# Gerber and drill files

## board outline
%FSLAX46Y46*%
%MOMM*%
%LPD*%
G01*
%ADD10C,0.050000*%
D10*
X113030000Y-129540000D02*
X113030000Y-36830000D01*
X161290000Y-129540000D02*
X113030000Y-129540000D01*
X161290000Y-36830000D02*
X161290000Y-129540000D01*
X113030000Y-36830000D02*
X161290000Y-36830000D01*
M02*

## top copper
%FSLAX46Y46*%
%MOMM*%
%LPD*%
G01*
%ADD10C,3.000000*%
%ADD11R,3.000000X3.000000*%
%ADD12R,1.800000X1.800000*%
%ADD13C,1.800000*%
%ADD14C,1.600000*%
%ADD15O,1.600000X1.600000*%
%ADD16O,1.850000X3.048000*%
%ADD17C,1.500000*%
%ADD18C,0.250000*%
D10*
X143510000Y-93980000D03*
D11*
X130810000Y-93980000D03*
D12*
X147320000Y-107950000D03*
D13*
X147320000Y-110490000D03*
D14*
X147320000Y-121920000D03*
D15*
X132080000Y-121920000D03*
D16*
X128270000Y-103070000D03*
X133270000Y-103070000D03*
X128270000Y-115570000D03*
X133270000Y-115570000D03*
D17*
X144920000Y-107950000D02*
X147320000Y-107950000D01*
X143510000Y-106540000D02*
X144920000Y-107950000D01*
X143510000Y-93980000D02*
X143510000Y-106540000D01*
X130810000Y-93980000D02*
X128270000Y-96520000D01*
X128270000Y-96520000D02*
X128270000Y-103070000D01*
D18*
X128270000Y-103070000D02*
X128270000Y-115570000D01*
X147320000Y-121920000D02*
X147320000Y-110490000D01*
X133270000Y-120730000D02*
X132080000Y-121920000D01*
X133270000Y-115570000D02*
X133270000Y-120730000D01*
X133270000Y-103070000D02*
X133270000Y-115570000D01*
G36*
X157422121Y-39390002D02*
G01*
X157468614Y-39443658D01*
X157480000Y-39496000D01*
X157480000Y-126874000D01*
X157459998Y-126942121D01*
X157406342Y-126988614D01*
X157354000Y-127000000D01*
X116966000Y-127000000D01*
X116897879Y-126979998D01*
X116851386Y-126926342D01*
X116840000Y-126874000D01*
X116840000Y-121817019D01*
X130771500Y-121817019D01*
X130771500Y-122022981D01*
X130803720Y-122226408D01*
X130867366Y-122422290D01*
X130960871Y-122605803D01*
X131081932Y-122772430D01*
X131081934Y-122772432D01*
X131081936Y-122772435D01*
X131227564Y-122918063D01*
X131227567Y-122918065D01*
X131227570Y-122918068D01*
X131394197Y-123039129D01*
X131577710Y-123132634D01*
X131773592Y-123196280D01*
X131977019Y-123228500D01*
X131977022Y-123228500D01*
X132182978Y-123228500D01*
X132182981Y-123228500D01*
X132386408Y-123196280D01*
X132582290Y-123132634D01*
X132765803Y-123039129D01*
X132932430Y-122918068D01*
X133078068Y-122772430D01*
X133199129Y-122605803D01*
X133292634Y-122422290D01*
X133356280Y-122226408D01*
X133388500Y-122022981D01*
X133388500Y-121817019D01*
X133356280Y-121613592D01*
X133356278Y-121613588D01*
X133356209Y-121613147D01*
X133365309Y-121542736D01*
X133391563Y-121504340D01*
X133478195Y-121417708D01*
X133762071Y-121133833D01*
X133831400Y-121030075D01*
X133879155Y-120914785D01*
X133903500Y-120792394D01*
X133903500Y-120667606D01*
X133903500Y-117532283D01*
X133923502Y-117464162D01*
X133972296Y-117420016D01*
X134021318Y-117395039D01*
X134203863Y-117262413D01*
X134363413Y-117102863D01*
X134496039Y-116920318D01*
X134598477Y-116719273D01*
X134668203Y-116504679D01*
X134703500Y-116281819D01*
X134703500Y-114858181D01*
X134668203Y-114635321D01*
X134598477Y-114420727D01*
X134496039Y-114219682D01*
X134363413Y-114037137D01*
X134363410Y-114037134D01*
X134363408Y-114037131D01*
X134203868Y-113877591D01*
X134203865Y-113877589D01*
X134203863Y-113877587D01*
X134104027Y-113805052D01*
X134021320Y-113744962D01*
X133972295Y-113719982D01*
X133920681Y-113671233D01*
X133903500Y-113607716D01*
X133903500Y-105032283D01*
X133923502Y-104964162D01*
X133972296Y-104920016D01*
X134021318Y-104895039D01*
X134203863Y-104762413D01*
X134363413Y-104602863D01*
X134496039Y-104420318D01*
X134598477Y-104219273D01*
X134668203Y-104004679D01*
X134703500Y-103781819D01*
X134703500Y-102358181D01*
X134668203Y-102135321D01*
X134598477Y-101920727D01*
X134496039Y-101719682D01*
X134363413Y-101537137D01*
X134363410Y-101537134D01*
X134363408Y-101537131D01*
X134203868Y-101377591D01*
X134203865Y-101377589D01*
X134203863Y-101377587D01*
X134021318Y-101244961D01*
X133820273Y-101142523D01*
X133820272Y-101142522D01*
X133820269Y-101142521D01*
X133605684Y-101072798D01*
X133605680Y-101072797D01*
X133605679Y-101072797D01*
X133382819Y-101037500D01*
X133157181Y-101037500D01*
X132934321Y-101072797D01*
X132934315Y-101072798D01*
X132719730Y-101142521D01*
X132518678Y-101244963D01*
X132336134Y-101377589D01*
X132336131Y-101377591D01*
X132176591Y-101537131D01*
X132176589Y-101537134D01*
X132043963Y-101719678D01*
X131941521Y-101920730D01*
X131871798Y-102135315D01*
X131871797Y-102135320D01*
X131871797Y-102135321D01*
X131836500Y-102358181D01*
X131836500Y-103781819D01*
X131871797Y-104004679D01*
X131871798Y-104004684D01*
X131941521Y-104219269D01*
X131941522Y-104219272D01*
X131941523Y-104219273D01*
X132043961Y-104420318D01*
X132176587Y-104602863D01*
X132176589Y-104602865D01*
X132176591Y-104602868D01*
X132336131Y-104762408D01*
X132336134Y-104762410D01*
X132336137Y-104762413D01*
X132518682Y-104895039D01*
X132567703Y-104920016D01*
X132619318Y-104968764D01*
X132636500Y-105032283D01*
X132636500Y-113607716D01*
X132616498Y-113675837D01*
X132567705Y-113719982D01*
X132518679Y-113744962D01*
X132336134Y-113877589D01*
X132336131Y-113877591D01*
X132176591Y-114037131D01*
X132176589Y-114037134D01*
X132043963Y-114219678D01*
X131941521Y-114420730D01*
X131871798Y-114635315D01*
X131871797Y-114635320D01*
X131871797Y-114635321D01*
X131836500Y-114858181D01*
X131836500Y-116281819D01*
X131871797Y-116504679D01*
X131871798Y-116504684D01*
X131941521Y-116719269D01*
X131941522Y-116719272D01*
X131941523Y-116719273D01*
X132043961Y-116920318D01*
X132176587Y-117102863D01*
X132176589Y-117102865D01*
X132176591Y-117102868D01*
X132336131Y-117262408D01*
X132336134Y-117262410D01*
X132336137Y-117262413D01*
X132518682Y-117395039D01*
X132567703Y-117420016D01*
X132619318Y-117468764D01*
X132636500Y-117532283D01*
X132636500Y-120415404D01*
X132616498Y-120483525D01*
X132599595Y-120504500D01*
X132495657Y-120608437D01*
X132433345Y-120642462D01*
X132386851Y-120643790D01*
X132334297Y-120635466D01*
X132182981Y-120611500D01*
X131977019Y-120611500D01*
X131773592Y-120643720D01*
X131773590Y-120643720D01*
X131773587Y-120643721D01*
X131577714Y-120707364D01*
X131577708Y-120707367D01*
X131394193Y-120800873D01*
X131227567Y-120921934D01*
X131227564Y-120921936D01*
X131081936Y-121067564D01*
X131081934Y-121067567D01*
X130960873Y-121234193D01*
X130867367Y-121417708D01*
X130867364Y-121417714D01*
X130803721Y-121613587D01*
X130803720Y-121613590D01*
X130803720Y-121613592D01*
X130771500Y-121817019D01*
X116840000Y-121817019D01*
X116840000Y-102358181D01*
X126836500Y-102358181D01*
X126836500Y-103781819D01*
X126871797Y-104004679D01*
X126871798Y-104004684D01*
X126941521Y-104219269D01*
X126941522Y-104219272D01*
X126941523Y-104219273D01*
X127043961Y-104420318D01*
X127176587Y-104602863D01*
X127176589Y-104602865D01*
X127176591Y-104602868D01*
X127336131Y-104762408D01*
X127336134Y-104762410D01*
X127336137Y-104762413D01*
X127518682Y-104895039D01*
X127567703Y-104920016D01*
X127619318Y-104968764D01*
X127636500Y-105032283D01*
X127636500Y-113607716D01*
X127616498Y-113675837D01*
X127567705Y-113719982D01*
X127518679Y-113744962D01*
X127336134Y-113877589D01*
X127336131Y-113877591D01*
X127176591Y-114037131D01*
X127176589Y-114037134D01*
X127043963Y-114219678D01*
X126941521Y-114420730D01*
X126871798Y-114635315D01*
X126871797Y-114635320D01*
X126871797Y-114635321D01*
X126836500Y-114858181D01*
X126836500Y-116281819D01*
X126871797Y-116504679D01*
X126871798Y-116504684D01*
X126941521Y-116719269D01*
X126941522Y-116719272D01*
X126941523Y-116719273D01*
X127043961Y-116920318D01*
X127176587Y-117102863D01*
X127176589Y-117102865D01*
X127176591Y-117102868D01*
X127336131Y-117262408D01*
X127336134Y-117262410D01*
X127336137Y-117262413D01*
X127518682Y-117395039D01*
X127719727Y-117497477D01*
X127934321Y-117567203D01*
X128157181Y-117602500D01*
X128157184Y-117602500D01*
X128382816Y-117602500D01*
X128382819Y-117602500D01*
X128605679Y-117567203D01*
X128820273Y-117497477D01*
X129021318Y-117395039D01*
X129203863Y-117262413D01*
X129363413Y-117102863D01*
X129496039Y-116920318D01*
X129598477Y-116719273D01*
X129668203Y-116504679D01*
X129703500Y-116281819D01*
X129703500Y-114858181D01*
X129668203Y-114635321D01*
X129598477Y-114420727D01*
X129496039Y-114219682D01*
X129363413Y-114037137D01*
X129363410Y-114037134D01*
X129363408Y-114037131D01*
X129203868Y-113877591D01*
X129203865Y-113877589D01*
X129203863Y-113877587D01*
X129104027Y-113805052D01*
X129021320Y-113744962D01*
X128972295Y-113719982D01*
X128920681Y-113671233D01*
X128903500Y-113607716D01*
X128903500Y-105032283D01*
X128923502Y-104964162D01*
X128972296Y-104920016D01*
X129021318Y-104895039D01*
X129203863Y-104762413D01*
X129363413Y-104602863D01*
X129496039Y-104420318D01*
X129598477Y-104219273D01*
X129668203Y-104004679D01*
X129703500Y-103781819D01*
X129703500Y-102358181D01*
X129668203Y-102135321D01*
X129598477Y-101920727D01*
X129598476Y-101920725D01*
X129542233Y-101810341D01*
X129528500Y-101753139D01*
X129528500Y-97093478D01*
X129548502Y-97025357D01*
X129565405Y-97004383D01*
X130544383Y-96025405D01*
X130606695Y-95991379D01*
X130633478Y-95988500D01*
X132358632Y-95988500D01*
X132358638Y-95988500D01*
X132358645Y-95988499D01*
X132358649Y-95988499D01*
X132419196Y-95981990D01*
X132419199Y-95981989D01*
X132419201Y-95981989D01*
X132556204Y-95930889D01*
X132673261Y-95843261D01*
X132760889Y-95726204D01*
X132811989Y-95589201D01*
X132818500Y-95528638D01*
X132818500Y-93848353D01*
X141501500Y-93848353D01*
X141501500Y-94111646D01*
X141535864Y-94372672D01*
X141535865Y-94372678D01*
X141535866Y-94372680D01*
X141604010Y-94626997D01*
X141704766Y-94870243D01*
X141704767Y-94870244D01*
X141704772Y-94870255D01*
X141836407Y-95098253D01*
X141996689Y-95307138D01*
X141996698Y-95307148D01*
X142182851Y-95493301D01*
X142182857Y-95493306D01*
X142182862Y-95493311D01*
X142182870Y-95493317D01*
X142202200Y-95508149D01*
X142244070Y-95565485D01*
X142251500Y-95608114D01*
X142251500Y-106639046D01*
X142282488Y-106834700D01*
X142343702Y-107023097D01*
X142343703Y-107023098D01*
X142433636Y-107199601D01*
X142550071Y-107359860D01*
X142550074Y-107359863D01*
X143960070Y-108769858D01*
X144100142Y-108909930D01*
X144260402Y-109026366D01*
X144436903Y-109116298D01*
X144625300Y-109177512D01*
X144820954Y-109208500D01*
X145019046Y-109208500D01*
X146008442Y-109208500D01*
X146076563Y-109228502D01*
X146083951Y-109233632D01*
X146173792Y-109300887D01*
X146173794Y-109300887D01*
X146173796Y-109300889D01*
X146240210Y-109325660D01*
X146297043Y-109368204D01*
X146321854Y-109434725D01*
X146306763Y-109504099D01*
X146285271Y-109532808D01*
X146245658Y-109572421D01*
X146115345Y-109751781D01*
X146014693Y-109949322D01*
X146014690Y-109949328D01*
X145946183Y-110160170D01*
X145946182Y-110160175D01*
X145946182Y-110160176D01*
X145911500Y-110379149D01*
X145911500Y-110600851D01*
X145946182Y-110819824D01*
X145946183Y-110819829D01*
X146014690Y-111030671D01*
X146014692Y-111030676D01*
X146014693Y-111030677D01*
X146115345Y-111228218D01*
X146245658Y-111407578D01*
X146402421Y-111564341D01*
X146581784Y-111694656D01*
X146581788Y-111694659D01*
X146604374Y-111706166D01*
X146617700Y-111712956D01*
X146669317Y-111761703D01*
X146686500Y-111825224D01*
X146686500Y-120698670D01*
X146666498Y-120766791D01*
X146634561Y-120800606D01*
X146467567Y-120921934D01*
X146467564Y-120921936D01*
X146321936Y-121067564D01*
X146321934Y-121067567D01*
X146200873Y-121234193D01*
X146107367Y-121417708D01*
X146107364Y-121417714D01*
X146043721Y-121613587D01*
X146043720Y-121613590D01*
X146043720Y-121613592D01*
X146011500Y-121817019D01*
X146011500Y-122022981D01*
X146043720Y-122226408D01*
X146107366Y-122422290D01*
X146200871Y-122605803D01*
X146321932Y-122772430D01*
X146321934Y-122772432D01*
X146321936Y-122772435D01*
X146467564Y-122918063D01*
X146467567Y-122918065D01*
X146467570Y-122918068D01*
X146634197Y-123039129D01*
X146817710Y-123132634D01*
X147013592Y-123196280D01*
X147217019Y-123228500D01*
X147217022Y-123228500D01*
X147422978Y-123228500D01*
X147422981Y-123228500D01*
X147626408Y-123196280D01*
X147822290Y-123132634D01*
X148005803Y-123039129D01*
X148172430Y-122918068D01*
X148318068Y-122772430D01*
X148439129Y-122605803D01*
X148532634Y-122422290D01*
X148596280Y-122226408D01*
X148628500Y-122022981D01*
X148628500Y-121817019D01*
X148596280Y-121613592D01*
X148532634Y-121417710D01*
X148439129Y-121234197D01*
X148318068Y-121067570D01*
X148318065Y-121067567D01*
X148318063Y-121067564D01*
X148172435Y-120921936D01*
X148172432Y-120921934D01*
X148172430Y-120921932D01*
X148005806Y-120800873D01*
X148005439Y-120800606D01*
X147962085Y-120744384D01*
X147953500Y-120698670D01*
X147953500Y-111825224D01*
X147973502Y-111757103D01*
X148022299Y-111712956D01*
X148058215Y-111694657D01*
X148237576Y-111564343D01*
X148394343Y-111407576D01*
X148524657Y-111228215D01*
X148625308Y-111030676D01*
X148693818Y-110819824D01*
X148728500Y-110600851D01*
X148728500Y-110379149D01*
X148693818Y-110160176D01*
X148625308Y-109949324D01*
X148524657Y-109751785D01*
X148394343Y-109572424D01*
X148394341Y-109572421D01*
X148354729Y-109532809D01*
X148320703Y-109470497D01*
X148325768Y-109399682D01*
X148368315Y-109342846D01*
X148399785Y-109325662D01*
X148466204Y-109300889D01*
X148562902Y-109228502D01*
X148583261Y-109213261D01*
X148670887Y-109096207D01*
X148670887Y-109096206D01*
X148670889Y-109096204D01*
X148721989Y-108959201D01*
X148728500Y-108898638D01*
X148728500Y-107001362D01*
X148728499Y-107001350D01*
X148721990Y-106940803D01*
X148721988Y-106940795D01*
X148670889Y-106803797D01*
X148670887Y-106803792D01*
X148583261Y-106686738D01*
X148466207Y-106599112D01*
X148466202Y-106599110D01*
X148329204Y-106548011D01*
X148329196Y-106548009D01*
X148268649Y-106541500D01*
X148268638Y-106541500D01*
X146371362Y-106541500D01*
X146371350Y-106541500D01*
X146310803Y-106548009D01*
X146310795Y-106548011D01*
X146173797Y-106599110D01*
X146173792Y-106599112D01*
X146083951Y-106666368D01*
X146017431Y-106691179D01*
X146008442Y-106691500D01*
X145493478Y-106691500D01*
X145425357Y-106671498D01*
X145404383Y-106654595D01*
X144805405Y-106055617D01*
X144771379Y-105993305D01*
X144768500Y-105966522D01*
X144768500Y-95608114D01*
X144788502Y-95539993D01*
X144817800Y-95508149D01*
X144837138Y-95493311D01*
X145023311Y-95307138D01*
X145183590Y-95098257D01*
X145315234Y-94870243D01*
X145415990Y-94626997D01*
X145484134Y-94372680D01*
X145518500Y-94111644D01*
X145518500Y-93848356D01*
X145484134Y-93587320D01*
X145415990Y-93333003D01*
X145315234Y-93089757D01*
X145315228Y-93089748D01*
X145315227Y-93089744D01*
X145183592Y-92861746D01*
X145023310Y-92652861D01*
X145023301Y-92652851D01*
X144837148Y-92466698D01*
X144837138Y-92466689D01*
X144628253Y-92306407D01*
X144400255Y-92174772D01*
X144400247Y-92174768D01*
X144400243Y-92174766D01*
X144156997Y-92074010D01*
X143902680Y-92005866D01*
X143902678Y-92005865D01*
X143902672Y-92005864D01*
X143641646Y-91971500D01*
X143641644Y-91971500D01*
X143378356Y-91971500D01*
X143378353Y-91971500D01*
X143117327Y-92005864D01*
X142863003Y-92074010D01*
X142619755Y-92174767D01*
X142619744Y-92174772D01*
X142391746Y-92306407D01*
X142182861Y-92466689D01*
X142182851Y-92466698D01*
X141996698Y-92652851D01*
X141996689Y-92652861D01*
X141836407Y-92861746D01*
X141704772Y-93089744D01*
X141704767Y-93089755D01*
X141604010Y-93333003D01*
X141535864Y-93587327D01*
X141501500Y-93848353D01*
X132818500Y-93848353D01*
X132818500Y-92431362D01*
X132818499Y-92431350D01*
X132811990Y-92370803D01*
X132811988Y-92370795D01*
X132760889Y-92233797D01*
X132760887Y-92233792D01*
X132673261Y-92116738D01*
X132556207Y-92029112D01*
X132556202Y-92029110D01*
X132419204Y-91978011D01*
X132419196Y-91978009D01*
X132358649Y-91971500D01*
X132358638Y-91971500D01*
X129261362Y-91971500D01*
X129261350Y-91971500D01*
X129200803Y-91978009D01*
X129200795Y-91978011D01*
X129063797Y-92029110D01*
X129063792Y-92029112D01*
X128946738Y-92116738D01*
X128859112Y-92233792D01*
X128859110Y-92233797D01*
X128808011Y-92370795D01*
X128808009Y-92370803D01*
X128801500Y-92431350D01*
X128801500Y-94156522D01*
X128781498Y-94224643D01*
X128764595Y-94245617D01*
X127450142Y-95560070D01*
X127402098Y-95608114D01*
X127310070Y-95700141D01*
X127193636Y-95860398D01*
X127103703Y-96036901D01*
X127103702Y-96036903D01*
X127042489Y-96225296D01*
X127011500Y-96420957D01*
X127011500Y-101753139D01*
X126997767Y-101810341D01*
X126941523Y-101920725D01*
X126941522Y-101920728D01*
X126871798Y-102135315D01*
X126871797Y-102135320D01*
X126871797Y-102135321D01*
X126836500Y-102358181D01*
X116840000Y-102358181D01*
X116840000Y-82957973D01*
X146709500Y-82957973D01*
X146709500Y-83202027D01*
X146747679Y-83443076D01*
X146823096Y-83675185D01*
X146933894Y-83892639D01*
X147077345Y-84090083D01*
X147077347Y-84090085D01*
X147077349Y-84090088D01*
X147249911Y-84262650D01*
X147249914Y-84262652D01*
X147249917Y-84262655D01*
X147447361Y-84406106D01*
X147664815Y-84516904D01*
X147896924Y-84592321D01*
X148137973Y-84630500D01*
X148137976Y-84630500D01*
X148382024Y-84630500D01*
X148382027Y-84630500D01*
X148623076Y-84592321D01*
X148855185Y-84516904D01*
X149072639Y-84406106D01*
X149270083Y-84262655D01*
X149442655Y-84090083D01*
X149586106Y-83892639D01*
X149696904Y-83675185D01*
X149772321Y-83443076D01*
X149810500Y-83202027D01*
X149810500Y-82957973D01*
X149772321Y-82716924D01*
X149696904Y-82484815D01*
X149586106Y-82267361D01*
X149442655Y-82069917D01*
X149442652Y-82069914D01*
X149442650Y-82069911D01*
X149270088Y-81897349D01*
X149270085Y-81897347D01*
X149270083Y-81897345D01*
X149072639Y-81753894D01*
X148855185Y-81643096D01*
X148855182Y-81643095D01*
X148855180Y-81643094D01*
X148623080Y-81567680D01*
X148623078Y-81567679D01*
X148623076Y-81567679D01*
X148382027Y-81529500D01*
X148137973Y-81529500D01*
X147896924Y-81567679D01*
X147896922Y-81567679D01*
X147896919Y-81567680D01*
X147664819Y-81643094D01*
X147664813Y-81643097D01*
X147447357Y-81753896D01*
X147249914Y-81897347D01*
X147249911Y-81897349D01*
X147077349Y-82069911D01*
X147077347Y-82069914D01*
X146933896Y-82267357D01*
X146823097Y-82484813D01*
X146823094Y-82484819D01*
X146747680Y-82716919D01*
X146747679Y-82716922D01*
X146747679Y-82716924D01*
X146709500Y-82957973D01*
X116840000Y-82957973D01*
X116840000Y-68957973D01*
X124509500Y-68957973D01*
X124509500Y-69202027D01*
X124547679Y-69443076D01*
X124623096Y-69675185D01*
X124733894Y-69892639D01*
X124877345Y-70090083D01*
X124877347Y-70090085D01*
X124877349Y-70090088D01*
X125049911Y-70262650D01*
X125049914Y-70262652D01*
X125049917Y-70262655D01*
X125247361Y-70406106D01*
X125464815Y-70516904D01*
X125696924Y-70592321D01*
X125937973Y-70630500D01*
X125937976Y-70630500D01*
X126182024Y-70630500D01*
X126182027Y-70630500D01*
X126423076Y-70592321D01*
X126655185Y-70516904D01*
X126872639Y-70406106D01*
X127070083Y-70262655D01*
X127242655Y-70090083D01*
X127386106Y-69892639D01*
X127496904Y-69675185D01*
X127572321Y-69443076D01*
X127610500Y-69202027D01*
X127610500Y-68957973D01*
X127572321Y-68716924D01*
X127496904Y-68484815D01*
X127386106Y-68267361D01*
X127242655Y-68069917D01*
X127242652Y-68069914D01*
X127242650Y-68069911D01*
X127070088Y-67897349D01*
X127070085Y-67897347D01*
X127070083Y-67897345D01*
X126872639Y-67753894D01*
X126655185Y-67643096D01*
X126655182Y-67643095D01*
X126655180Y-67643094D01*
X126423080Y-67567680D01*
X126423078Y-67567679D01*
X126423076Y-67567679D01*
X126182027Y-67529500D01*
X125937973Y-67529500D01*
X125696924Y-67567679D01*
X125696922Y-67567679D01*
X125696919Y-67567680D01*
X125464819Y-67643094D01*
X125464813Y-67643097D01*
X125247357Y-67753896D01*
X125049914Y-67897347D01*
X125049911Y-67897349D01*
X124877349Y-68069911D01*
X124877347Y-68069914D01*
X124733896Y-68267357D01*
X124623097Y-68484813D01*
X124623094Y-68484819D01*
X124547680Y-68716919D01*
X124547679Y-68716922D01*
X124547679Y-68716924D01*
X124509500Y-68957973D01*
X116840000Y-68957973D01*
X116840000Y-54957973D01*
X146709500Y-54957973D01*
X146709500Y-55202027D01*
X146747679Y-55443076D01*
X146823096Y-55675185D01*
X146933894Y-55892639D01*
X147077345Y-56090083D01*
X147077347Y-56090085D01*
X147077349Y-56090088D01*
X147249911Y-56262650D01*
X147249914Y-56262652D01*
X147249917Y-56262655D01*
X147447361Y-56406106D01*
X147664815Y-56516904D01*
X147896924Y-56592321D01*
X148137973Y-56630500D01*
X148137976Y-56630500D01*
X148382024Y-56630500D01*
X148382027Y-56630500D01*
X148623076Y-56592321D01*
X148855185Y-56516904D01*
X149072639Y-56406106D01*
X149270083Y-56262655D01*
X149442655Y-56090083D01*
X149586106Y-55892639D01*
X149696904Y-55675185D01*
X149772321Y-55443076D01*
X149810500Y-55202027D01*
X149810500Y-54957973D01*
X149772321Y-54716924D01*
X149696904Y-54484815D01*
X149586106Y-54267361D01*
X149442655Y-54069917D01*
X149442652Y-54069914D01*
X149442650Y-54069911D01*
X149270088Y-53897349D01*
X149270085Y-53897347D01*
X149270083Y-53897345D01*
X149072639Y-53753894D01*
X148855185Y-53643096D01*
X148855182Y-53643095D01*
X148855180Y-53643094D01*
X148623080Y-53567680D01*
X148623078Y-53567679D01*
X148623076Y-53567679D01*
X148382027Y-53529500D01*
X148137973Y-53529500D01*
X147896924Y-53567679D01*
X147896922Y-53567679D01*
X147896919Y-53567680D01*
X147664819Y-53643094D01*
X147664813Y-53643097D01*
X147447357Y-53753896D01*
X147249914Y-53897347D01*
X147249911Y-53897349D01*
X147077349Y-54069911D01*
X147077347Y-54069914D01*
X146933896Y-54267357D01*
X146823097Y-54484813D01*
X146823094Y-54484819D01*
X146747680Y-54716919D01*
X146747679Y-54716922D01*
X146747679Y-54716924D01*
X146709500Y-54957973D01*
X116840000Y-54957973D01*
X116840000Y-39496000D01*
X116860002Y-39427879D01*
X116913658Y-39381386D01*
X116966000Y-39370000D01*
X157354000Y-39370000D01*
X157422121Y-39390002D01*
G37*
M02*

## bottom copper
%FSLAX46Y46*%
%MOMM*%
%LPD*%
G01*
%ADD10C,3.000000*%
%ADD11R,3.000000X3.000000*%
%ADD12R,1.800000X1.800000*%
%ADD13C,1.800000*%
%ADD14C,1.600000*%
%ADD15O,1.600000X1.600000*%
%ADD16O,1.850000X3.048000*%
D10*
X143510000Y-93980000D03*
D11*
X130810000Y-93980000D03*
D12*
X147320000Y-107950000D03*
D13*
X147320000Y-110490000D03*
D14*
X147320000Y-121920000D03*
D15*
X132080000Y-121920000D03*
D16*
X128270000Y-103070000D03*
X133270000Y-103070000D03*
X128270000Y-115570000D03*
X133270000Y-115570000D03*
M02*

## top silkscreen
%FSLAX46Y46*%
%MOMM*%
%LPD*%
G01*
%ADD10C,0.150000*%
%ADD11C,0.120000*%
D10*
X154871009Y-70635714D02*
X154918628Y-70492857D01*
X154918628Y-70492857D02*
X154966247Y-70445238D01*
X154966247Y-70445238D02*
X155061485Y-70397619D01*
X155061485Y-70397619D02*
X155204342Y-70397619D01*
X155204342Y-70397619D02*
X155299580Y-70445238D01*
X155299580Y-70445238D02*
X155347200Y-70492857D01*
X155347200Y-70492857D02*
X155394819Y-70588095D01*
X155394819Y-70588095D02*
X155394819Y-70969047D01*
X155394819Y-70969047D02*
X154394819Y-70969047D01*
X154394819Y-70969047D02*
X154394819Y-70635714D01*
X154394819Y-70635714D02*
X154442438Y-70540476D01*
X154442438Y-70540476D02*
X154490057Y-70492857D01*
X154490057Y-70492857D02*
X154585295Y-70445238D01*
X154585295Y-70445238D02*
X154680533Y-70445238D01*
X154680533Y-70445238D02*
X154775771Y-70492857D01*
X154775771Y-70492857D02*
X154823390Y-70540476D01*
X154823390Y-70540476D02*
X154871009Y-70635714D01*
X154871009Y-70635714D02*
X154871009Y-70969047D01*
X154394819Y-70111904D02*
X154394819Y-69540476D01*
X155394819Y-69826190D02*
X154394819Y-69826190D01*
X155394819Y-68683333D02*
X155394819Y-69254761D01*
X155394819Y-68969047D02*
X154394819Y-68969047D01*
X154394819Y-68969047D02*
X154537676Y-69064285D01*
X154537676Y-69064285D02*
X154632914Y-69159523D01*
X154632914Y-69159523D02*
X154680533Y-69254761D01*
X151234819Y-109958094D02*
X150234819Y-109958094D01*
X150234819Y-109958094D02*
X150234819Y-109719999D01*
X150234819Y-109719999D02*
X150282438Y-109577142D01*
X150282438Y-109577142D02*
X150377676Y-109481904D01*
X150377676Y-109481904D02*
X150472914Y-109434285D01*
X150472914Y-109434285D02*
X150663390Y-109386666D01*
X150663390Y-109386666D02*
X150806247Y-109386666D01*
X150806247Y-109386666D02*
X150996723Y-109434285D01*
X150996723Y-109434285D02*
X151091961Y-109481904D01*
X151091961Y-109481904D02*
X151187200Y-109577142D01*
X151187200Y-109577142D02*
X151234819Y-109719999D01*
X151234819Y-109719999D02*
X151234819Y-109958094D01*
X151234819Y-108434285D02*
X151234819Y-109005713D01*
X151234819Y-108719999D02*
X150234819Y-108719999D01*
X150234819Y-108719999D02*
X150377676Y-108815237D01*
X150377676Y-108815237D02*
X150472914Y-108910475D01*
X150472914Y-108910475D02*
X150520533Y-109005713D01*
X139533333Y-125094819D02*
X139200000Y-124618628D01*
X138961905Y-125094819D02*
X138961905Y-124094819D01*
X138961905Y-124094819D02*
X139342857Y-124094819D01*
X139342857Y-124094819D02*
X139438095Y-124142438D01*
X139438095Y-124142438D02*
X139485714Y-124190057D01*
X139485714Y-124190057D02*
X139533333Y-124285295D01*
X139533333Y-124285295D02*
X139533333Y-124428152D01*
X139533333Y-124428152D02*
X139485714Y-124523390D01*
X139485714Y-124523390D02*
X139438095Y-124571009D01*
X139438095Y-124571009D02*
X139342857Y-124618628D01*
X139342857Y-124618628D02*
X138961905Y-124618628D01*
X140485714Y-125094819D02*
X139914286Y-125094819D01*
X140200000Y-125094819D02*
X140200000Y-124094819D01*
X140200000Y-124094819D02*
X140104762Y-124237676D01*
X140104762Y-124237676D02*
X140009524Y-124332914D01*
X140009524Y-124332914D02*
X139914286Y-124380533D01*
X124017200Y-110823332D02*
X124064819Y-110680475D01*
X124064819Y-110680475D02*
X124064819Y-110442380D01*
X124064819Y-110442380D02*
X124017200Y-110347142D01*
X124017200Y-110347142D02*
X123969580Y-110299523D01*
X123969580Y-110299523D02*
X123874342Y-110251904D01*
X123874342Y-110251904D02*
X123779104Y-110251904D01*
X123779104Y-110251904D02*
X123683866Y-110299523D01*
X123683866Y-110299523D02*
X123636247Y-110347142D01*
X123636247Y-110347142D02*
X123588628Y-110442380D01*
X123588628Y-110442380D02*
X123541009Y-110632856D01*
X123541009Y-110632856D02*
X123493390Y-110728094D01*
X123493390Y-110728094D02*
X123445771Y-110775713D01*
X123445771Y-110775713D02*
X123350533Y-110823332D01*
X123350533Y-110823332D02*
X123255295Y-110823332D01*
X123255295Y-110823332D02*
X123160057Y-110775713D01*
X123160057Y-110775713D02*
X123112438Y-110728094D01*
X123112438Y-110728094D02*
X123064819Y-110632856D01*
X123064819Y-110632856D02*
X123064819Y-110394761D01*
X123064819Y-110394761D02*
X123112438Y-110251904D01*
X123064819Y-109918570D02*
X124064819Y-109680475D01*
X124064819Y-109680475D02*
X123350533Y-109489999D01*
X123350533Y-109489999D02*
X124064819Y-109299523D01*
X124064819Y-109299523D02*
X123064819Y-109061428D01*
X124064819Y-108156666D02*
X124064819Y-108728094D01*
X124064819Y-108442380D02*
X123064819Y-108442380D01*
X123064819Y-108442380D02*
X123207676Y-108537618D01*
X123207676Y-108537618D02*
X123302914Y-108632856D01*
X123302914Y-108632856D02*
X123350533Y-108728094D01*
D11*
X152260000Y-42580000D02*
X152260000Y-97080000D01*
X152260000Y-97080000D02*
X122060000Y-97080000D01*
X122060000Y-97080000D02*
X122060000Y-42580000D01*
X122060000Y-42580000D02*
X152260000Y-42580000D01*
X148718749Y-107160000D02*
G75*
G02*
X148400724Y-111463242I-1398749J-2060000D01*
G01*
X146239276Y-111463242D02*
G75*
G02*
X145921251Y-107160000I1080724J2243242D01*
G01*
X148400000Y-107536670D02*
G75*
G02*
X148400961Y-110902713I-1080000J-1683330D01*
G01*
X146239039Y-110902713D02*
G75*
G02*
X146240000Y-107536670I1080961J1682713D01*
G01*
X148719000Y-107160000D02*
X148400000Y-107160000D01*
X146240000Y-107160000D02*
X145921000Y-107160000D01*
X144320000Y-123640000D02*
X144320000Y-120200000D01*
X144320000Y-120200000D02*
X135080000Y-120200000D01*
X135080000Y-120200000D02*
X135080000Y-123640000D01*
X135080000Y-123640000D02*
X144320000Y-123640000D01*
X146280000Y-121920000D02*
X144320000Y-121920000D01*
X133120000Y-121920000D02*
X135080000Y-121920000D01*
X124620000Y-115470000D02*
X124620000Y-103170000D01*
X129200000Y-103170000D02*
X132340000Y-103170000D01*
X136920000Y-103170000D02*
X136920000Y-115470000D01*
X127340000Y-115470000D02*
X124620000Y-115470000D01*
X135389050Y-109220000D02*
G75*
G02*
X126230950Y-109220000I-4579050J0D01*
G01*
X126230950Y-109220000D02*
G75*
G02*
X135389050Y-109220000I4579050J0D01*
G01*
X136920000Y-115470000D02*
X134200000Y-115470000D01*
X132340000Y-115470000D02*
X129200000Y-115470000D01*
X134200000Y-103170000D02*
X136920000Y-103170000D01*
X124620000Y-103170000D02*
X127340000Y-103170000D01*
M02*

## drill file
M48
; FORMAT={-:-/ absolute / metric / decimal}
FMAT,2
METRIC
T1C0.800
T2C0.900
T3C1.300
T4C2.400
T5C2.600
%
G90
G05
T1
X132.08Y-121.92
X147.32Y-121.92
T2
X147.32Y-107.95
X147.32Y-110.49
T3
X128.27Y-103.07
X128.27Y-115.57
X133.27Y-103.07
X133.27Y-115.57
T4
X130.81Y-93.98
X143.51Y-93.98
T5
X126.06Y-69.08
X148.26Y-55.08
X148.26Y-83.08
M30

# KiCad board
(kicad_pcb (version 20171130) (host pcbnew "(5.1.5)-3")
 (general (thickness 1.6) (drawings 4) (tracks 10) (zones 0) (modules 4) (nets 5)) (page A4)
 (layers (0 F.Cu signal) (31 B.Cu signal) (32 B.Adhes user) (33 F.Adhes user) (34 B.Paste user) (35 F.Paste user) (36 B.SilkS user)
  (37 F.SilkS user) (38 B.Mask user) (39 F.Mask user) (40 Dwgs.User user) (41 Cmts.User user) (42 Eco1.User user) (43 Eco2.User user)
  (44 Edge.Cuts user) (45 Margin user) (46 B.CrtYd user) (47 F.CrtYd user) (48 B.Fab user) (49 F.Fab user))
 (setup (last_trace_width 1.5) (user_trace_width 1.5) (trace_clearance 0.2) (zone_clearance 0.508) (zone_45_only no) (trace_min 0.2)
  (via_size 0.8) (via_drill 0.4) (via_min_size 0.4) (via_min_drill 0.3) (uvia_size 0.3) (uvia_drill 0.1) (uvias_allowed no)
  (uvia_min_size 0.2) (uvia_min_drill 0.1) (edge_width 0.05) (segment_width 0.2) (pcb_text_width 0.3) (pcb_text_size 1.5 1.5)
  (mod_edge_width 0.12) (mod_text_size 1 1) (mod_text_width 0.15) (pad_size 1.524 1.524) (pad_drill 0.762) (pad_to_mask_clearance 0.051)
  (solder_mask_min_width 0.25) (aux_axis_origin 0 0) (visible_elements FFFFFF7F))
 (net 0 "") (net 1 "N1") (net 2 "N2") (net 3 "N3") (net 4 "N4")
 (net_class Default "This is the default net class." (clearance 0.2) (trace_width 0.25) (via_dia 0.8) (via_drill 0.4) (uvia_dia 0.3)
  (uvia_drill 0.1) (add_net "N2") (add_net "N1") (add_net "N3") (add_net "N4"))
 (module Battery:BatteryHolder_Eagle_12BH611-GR (layer F.Cu) (at 130.81 93.98 270)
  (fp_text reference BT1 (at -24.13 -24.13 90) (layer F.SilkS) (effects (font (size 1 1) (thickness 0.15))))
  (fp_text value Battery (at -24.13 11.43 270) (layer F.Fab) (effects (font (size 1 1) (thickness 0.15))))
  (fp_line (start -51.4 -21.45) (end 3.1 -21.45) (layer F.SilkS) (width 0.12))
  (fp_line (start 3.1 -21.45) (end 3.1 8.75) (layer F.SilkS) (width 0.12))
  (fp_line (start 3.1 8.75) (end -51.4 8.75) (layer F.SilkS) (width 0.12))
  (fp_line (start -51.4 8.75) (end -51.4 -21.45) (layer F.SilkS) (width 0.12))
  (pad 2 thru_hole circle (at 0 -12.7 270) (size 3 3) (drill 2.4) (layers *.Cu *.Mask) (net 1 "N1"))
  (pad 1 thru_hole rect (at 0 0 270) (size 3 3) (drill 2.4) (layers *.Cu *.Mask) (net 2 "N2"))
  (pad "" np_thru_hole circle (at -10.9 -17.45 270) (size 2.6 2.6) (drill 2.6) (layers *.Cu *.Mask))
  (pad "" np_thru_hole circle (at -38.9 -17.45 270) (size 2.6 2.6) (drill 2.6) (layers *.Cu *.Mask))
  (pad "" np_thru_hole circle (at -24.9 4.75 270) (size 2.6 2.6) (drill 2.6) (layers *.Cu *.Mask)))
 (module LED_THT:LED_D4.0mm (layer F.Cu) (at 147.32 107.95 270)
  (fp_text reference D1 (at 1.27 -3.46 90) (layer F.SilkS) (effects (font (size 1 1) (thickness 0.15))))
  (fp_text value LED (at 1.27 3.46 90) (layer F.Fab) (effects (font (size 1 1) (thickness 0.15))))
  (fp_arc (start 1.27 0) (end -0.79 -1.398749) (angle 120.1) (layer F.SilkS) (width 0.12))
  (fp_arc (start 1.27 0) (end -0.79 1.398749) (angle -120.1) (layer F.SilkS) (width 0.12))
  (fp_arc (start 1.27 0) (end -0.41333 -1.08) (angle 114.6) (layer F.SilkS) (width 0.12))
  (fp_arc (start 1.27 0) (end -0.41333 1.08) (angle -114.6) (layer F.SilkS) (width 0.12))
  (fp_line (start -0.79 -1.399) (end -0.79 -1.08) (layer F.SilkS) (width 0.12))
  (fp_line (start -0.79 1.08) (end -0.79 1.399) (layer F.SilkS) (width 0.12))
  (pad 1 thru_hole rect (at 0 0 270) (size 1.8 1.8) (drill 0.9) (layers *.Cu *.Mask) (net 1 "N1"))
  (pad 2 thru_hole circle (at 2.54 0 270) (size 1.8 1.8) (drill 0.9) (layers *.Cu *.Mask) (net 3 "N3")))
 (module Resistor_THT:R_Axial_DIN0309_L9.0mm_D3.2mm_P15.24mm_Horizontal (layer F.Cu) (at 147.32 121.92 180)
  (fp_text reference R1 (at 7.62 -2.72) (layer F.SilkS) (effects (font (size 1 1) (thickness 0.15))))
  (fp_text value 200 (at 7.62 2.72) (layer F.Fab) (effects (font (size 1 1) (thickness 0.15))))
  (fp_line (start 3 -1.72) (end 3 1.72) (layer F.SilkS) (width 0.12))
  (fp_line (start 3 1.72) (end 12.24 1.72) (layer F.SilkS) (width 0.12))
  (fp_line (start 12.24 1.72) (end 12.24 -1.72) (layer F.SilkS) (width 0.12))
  (fp_line (start 12.24 -1.72) (end 3 -1.72) (layer F.SilkS) (width 0.12))
  (fp_line (start 1.04 0) (end 3 0) (layer F.SilkS) (width 0.12))
  (fp_line (start 14.2 0) (end 12.24 0) (layer F.SilkS) (width 0.12))
  (pad 1 thru_hole circle (at 0 0 180) (size 1.6 1.6) (drill 0.8) (layers *.Cu *.Mask) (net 3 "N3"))
  (pad 2 thru_hole oval (at 15.24 0 180) (size 1.6 1.6) (drill 0.8) (layers *.Cu *.Mask) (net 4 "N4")))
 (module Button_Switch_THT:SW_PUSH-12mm (layer F.Cu) (at 128.27 115.57 90)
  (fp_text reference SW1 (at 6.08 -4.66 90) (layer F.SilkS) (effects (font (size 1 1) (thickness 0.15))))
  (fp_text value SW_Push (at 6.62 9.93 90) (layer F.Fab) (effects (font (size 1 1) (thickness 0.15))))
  (fp_line (start 0.1 -3.65) (end 12.4 -3.65) (layer F.SilkS) (width 0.12))
  (fp_line (start 12.4 0.93) (end 12.4 4.07) (layer F.SilkS) (width 0.12))
  (fp_line (start 12.4 8.65) (end 0.1 8.65) (layer F.SilkS) (width 0.12))
  (fp_line (start 0.1 -0.93) (end 0.1 -3.65) (layer F.SilkS) (width 0.12))
  (fp_circle (center 6.35 2.54) (end 10.16 5.08) (layer F.SilkS) (width 0.12))
  (fp_line (start 0.1 8.65) (end 0.1 5.93) (layer F.SilkS) (width 0.12))
  (fp_line (start 0.1 4.07) (end 0.1 0.93) (layer F.SilkS) (width 0.12))
  (fp_line (start 12.4 5.93) (end 12.4 8.65) (layer F.SilkS) (width 0.12))
  (fp_line (start 12.4 -3.65) (end 12.4 -0.93) (layer F.SilkS) (width 0.12))
  (pad 1 thru_hole oval (at 12.5 0 90) (size 3.048 1.85) (drill 1.3) (layers *.Cu *.Mask) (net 2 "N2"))
  (pad 2 thru_hole oval (at 12.5 5 90) (size 3.048 1.85) (drill 1.3) (layers *.Cu *.Mask) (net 4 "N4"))
  (pad 1 thru_hole oval (at 0 0 90) (size 3.048 1.85) (drill 1.3) (layers *.Cu *.Mask) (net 2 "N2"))
  (pad 2 thru_hole oval (at 0 5 90) (size 3.048 1.85) (drill 1.3) (layers *.Cu *.Mask) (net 4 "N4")))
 (gr_line (start 113.03 129.54) (end 113.03 36.83) (layer Edge.Cuts) (width 0.05))
 (gr_line (start 161.29 129.54) (end 113.03 129.54) (layer Edge.Cuts) (width 0.05))
 (gr_line (start 161.29 36.83) (end 161.29 129.54) (layer Edge.Cuts) (width 0.05))
 (gr_line (start 113.03 36.83) (end 161.29 36.83) (layer Edge.Cuts) (width 0.05))
 (segment (start 144.92 107.95) (end 147.32 107.95) (width 1.5) (layer F.Cu) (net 1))
 (segment (start 143.51 106.54) (end 144.92 107.95) (width 1.5) (layer F.Cu) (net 1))
 (segment (start 143.51 93.98) (end 143.51 106.54) (width 1.5) (layer F.Cu) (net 1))
 (segment (start 130.81 93.98) (end 128.27 96.52) (width 1.5) (layer F.Cu) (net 2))
 (segment (start 128.27 96.52) (end 128.27 103.07) (width 1.5) (layer F.Cu) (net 2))
 (segment (start 128.27 103.07) (end 128.27 115.57) (width 0.25) (layer F.Cu) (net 2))
 (segment (start 147.32 121.92) (end 147.32 110.49) (width 0.25) (layer F.Cu) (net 3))
 (segment (start 133.27 120.73) (end 132.08 121.92) (width 0.25) (layer F.Cu) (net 4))
 (segment (start 133.27 115.57) (end 133.27 120.73) (width 0.25) (layer F.Cu) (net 4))
 (segment (start 133.27 103.07) (end 133.27 115.57) (width 0.25) (layer F.Cu) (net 4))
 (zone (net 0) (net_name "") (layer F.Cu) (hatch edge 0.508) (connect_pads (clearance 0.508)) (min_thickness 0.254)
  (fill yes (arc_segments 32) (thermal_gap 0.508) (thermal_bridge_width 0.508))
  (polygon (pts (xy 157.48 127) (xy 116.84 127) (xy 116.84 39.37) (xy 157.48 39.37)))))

